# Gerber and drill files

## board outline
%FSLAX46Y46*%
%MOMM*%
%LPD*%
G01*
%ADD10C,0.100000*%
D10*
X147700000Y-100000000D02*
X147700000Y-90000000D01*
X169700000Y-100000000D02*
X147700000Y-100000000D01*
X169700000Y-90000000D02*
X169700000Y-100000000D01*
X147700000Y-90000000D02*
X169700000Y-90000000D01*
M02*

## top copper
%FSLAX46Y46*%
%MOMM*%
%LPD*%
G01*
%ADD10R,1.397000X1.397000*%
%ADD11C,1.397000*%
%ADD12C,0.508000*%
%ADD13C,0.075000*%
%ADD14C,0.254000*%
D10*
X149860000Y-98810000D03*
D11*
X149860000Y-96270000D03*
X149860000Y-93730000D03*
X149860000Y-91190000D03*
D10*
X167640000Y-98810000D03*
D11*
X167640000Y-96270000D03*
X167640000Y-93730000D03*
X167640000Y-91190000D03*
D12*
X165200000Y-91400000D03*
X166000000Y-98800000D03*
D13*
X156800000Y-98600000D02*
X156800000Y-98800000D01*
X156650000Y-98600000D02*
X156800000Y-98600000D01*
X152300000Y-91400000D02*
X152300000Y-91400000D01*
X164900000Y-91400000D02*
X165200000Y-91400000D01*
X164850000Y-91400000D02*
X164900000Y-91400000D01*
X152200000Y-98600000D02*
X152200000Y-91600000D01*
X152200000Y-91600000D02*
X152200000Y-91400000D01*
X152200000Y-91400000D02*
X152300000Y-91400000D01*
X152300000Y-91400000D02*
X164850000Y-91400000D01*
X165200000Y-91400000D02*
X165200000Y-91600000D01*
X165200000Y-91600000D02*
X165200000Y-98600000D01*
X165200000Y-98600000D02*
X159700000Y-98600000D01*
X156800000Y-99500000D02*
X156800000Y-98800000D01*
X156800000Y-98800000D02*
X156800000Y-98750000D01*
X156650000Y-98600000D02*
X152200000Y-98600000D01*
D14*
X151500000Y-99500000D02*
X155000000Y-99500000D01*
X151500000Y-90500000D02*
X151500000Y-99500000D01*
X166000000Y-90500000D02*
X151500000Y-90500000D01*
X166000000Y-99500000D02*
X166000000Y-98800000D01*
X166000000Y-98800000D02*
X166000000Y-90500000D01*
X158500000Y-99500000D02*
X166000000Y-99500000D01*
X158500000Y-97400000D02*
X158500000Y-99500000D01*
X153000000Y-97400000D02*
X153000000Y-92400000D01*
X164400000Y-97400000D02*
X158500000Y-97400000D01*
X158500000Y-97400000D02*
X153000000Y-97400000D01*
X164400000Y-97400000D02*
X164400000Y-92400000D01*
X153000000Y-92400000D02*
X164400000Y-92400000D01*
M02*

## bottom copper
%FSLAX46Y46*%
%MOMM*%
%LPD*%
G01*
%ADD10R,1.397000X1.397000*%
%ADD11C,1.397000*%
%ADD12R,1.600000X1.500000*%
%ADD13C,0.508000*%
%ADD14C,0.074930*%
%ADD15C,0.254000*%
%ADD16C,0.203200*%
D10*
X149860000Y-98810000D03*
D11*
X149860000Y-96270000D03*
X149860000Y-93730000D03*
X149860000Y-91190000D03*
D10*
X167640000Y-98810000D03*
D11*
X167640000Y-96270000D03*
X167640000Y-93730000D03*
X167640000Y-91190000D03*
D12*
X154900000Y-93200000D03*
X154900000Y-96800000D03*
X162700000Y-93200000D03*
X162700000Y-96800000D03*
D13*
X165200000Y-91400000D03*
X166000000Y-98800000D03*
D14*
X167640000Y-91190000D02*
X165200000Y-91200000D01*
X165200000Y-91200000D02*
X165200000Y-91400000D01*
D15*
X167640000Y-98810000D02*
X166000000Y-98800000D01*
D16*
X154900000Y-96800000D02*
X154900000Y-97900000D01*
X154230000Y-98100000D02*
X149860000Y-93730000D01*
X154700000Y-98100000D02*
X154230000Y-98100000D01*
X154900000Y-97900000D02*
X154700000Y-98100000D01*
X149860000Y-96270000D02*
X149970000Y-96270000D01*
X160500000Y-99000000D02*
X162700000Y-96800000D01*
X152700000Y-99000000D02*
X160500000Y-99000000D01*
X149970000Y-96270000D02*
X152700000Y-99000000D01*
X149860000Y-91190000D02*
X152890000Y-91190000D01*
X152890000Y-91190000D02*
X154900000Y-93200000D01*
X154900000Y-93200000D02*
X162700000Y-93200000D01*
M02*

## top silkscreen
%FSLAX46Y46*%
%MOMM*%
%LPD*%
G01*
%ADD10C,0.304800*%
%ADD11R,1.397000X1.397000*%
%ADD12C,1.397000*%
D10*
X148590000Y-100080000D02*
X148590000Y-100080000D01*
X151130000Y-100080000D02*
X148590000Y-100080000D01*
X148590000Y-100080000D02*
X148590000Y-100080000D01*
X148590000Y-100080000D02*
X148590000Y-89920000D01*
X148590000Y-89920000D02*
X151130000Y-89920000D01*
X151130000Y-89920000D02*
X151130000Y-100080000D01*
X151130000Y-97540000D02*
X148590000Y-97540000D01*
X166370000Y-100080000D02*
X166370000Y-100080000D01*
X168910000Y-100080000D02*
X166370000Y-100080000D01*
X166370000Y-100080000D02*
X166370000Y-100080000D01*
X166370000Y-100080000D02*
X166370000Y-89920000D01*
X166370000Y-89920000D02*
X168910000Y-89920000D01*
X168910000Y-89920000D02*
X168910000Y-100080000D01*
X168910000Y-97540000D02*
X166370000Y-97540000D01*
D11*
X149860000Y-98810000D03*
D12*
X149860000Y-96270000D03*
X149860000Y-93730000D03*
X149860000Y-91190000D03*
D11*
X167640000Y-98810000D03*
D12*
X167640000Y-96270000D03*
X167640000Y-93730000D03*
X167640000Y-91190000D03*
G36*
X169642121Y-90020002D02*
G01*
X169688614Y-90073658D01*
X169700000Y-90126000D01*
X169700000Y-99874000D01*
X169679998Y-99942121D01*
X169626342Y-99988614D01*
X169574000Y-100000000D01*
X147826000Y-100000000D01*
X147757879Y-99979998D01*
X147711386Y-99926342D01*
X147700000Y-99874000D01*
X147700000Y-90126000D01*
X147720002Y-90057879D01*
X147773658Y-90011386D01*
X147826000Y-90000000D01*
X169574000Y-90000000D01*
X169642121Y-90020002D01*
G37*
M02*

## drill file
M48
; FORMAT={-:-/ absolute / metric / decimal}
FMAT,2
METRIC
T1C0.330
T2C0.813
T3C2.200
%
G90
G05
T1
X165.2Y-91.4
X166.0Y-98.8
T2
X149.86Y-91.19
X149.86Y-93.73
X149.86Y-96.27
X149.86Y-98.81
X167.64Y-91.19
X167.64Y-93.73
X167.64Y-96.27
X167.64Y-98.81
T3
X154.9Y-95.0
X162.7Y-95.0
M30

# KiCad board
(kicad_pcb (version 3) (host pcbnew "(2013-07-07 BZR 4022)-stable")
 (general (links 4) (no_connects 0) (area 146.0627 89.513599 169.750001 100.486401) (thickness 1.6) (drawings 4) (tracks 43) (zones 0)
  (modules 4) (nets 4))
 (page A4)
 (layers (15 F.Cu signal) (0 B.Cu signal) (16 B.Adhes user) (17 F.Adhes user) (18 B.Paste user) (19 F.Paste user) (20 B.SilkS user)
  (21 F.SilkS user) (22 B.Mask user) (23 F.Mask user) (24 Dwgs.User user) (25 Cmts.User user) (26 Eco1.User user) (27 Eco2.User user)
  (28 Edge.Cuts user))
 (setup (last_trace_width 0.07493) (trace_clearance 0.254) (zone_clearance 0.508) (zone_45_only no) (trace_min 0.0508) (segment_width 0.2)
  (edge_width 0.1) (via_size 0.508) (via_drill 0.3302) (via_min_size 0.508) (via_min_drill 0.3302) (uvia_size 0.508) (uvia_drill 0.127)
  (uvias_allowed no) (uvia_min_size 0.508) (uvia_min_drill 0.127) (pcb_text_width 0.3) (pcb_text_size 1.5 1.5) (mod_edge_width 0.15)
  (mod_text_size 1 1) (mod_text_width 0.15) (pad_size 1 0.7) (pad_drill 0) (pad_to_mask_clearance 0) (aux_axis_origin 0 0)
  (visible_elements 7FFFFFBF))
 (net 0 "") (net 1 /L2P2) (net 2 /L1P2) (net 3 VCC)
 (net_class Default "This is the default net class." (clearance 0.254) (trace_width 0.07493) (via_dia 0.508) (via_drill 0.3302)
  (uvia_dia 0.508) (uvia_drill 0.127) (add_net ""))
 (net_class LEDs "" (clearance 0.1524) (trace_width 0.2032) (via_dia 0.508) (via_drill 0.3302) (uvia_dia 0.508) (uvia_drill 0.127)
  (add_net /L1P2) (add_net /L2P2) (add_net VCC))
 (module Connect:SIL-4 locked (layer F.Cu) (at 149.86 95 90)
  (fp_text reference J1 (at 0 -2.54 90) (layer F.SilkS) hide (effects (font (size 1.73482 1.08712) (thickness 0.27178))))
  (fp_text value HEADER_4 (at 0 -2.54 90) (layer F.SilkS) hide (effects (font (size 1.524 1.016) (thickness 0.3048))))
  (fp_line (start -5.08 -1.27) (end -5.08 -1.27) (layer F.SilkS) (width 0.3048))
  (fp_line (start -5.08 1.27) (end -5.08 -1.27) (layer F.SilkS) (width 0.3048))
  (fp_line (start -5.08 -1.27) (end -5.08 -1.27) (layer F.SilkS) (width 0.3048))
  (fp_line (start -5.08 -1.27) (end 5.08 -1.27) (layer F.SilkS) (width 0.3048))
  (fp_line (start 5.08 -1.27) (end 5.08 1.27) (layer F.SilkS) (width 0.3048))
  (fp_line (start 5.08 1.27) (end -5.08 1.27) (layer F.SilkS) (width 0.3048))
  (fp_line (start -2.54 1.27) (end -2.54 -1.27) (layer F.SilkS) (width 0.3048))
  (pad 1 thru_hole rect (at -3.81 0 90) (size 1.397 1.397) (drill 0.8128) (layers *.Cu *.Mask F.SilkS))
  (pad 2 thru_hole circle (at -1.27 0 90) (size 1.397 1.397) (drill 0.8128) (layers *.Cu *.Mask F.SilkS) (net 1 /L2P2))
  (pad 3 thru_hole circle (at 1.27 0 90) (size 1.397 1.397) (drill 0.8128) (layers *.Cu *.Mask F.SilkS) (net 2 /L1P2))
  (pad 4 thru_hole circle (at 3.81 0 90) (size 1.397 1.397) (drill 0.8128) (layers *.Cu *.Mask F.SilkS) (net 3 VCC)))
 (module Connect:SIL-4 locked (layer F.Cu) (at 167.64 95 90)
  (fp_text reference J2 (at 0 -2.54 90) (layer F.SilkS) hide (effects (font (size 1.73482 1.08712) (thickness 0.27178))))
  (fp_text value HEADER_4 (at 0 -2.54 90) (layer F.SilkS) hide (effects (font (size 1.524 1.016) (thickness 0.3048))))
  (fp_line (start -5.08 -1.27) (end -5.08 -1.27) (layer F.SilkS) (width 0.3048))
  (fp_line (start -5.08 1.27) (end -5.08 -1.27) (layer F.SilkS) (width 0.3048))
  (fp_line (start -5.08 -1.27) (end -5.08 -1.27) (layer F.SilkS) (width 0.3048))
  (fp_line (start -5.08 -1.27) (end 5.08 -1.27) (layer F.SilkS) (width 0.3048))
  (fp_line (start 5.08 -1.27) (end 5.08 1.27) (layer F.SilkS) (width 0.3048))
  (fp_line (start 5.08 1.27) (end -5.08 1.27) (layer F.SilkS) (width 0.3048))
  (fp_line (start -2.54 1.27) (end -2.54 -1.27) (layer F.SilkS) (width 0.3048))
  (pad 1 thru_hole rect (at -3.81 0 90) (size 1.397 1.397) (drill 0.8128) (layers *.Cu *.Mask F.SilkS))
  (pad 2 thru_hole circle (at -1.27 0 90) (size 1.397 1.397) (drill 0.8128) (layers *.Cu *.Mask F.SilkS))
  (pad 3 thru_hole circle (at 1.27 0 90) (size 1.397 1.397) (drill 0.8128) (layers *.Cu *.Mask F.SilkS))
  (pad 4 thru_hole circle (at 3.81 0 90) (size 1.397 1.397) (drill 0.8128) (layers *.Cu *.Mask F.SilkS)))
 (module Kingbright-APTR (layer B.Cu) (at 154.9 95 270)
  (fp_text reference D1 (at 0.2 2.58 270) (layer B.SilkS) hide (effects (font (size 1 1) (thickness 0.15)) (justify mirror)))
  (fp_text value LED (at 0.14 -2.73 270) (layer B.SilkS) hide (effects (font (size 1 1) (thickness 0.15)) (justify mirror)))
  (pad "" np_thru_hole circle (at 0 0 270) (size 2.2 2.2) (drill 2.2) (layers *.Cu *.Mask B.SilkS))
  (pad 1 smd rect (at -1.8 0 270) (size 1.5 1.6) (layers B.Cu B.Paste B.Mask) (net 3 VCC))
  (pad 2 smd rect (at 1.8 0 270) (size 1.5 1.6) (layers B.Cu B.Paste B.Mask) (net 2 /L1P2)))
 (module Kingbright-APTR (layer B.Cu) (at 162.7 95 270)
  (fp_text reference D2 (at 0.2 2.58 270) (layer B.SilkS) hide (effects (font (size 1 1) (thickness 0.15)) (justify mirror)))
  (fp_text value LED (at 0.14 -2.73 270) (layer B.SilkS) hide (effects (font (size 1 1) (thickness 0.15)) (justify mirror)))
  (pad "" np_thru_hole circle (at 0 0 270) (size 2.2 2.2) (drill 2.2) (layers *.Cu *.Mask B.SilkS))
  (pad 1 smd rect (at -1.8 0 270) (size 1.5 1.6) (layers B.Cu B.Paste B.Mask) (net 3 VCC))
  (pad 2 smd rect (at 1.8 0 270) (size 1.5 1.6) (layers B.Cu B.Paste B.Mask) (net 1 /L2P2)))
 (gr_line (start 147.7 100) (end 147.7 90) (angle 90) (layer Edge.Cuts) (width 0.1))
 (gr_line (start 169.7 100) (end 147.7 100) (angle 90) (layer Edge.Cuts) (width 0.1))
 (gr_line (start 169.7 90) (end 169.7 100) (angle 90) (layer Edge.Cuts) (width 0.1))
 (gr_line (start 147.7 90) (end 169.7 90) (angle 90) (layer Edge.Cuts) (width 0.1))
 (segment (start 167.64 91.19) (end 165.2 91.2) (width 0.07493) (layer B.Cu) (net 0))
 (segment (start 165.2 91.2) (end 165.2 91.4) (width 0.07493) (layer B.Cu) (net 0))
 (via (at 165.2 91.4) (size 0.508) (layers F.Cu B.Cu) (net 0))
 (segment (start 167.64 98.81) (end 166 98.8) (width 0.254) (layer B.Cu) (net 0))
 (via (at 166 98.8) (size 0.508) (layers F.Cu B.Cu) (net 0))
 (segment (start 156.8 98.6) (end 156.8 98.8) (width 0.075) (layer F.Cu) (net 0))
 (segment (start 156.65 98.6) (end 156.8 98.6) (width 0.075) (layer F.Cu) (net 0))
 (segment (start 152.3 91.4) (end 152.3 91.4) (width 0.075) (layer F.Cu) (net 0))
 (segment (start 164.9 91.4) (end 165.2 91.4) (width 0.075) (layer F.Cu) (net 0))
 (segment (start 164.85 91.4) (end 164.9 91.4) (width 0.075) (layer F.Cu) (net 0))
 (segment (start 152.2 98.6) (end 152.2 91.6) (width 0.075) (layer F.Cu) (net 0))
 (segment (start 152.2 91.6) (end 152.2 91.4) (width 0.075) (layer F.Cu) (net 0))
 (segment (start 152.2 91.4) (end 152.3 91.4) (width 0.075) (layer F.Cu) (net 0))
 (segment (start 152.3 91.4) (end 164.85 91.4) (width 0.075) (layer F.Cu) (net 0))
 (segment (start 165.2 91.4) (end 165.2 91.6) (width 0.075) (layer F.Cu) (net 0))
 (segment (start 165.2 91.6) (end 165.2 98.6) (width 0.075) (layer F.Cu) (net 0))
 (segment (start 165.2 98.6) (end 159.7 98.6) (width 0.075) (layer F.Cu) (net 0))
 (segment (start 156.8 99.5) (end 156.8 98.8) (width 0.075) (layer F.Cu) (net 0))
 (segment (start 156.8 98.8) (end 156.8 98.75) (width 0.075) (layer F.Cu) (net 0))
 (segment (start 156.65 98.6) (end 152.2 98.6) (width 0.075) (layer F.Cu) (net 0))
 (segment (start 151.5 99.5) (end 155 99.5) (width 0.254) (layer F.Cu) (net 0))
 (segment (start 151.5 90.5) (end 151.5 99.5) (width 0.254) (layer F.Cu) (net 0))
 (segment (start 166 90.5) (end 151.5 90.5) (width 0.254) (layer F.Cu) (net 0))
 (segment (start 166 99.5) (end 166 98.8) (width 0.254) (layer F.Cu) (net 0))
 (segment (start 166 98.8) (end 166 90.5) (width 0.254) (layer F.Cu) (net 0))
 (segment (start 158.5 99.5) (end 166 99.5) (width 0.254) (layer F.Cu) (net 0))
 (segment (start 158.5 97.4) (end 158.5 99.5) (width 0.254) (layer F.Cu) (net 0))
 (segment (start 153 97.4) (end 153 92.4) (width 0.254) (layer F.Cu) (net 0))
 (segment (start 164.4 97.4) (end 158.5 97.4) (width 0.254) (layer F.Cu) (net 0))
 (segment (start 158.5 97.4) (end 153 97.4) (width 0.254) (layer F.Cu) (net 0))
 (segment (start 164.4 97.4) (end 164.4 92.4) (width 0.254) (layer F.Cu) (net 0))
 (segment (start 153 92.4) (end 164.4 92.4) (width 0.254) (layer F.Cu) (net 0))
 (segment (start 154.9 96.8) (end 154.9 97.9) (width 0.2032) (layer B.Cu) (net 2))
 (segment (start 154.23 98.1) (end 149.86 93.73) (width 0.2032) (layer B.Cu) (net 2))
 (segment (start 154.7 98.1) (end 154.23 98.1) (width 0.2032) (layer B.Cu) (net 2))
 (segment (start 154.9 97.9) (end 154.7 98.1) (width 0.2032) (layer B.Cu) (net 2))
 (segment (start 149.86 96.27) (end 149.97 96.27) (width 0.2032) (layer B.Cu) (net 1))
 (segment (start 160.5 99) (end 162.7 96.8) (width 0.2032) (layer B.Cu) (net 1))
 (segment (start 152.7 99) (end 160.5 99) (width 0.2032) (layer B.Cu) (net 1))
 (segment (start 149.97 96.27) (end 152.7 99) (width 0.2032) (layer B.Cu) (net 1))
 (segment (start 149.86 91.19) (end 152.89 91.19) (width 0.2032) (layer B.Cu) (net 3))
 (segment (start 152.89 91.19) (end 154.9 93.2) (width 0.2032) (layer B.Cu) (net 3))
 (segment (start 154.9 93.2) (end 162.7 93.2) (width 0.2032) (layer B.Cu) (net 3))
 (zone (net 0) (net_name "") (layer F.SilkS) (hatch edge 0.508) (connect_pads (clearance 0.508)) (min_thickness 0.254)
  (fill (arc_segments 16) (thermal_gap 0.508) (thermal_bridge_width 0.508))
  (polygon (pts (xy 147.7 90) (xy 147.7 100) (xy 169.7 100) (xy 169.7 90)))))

